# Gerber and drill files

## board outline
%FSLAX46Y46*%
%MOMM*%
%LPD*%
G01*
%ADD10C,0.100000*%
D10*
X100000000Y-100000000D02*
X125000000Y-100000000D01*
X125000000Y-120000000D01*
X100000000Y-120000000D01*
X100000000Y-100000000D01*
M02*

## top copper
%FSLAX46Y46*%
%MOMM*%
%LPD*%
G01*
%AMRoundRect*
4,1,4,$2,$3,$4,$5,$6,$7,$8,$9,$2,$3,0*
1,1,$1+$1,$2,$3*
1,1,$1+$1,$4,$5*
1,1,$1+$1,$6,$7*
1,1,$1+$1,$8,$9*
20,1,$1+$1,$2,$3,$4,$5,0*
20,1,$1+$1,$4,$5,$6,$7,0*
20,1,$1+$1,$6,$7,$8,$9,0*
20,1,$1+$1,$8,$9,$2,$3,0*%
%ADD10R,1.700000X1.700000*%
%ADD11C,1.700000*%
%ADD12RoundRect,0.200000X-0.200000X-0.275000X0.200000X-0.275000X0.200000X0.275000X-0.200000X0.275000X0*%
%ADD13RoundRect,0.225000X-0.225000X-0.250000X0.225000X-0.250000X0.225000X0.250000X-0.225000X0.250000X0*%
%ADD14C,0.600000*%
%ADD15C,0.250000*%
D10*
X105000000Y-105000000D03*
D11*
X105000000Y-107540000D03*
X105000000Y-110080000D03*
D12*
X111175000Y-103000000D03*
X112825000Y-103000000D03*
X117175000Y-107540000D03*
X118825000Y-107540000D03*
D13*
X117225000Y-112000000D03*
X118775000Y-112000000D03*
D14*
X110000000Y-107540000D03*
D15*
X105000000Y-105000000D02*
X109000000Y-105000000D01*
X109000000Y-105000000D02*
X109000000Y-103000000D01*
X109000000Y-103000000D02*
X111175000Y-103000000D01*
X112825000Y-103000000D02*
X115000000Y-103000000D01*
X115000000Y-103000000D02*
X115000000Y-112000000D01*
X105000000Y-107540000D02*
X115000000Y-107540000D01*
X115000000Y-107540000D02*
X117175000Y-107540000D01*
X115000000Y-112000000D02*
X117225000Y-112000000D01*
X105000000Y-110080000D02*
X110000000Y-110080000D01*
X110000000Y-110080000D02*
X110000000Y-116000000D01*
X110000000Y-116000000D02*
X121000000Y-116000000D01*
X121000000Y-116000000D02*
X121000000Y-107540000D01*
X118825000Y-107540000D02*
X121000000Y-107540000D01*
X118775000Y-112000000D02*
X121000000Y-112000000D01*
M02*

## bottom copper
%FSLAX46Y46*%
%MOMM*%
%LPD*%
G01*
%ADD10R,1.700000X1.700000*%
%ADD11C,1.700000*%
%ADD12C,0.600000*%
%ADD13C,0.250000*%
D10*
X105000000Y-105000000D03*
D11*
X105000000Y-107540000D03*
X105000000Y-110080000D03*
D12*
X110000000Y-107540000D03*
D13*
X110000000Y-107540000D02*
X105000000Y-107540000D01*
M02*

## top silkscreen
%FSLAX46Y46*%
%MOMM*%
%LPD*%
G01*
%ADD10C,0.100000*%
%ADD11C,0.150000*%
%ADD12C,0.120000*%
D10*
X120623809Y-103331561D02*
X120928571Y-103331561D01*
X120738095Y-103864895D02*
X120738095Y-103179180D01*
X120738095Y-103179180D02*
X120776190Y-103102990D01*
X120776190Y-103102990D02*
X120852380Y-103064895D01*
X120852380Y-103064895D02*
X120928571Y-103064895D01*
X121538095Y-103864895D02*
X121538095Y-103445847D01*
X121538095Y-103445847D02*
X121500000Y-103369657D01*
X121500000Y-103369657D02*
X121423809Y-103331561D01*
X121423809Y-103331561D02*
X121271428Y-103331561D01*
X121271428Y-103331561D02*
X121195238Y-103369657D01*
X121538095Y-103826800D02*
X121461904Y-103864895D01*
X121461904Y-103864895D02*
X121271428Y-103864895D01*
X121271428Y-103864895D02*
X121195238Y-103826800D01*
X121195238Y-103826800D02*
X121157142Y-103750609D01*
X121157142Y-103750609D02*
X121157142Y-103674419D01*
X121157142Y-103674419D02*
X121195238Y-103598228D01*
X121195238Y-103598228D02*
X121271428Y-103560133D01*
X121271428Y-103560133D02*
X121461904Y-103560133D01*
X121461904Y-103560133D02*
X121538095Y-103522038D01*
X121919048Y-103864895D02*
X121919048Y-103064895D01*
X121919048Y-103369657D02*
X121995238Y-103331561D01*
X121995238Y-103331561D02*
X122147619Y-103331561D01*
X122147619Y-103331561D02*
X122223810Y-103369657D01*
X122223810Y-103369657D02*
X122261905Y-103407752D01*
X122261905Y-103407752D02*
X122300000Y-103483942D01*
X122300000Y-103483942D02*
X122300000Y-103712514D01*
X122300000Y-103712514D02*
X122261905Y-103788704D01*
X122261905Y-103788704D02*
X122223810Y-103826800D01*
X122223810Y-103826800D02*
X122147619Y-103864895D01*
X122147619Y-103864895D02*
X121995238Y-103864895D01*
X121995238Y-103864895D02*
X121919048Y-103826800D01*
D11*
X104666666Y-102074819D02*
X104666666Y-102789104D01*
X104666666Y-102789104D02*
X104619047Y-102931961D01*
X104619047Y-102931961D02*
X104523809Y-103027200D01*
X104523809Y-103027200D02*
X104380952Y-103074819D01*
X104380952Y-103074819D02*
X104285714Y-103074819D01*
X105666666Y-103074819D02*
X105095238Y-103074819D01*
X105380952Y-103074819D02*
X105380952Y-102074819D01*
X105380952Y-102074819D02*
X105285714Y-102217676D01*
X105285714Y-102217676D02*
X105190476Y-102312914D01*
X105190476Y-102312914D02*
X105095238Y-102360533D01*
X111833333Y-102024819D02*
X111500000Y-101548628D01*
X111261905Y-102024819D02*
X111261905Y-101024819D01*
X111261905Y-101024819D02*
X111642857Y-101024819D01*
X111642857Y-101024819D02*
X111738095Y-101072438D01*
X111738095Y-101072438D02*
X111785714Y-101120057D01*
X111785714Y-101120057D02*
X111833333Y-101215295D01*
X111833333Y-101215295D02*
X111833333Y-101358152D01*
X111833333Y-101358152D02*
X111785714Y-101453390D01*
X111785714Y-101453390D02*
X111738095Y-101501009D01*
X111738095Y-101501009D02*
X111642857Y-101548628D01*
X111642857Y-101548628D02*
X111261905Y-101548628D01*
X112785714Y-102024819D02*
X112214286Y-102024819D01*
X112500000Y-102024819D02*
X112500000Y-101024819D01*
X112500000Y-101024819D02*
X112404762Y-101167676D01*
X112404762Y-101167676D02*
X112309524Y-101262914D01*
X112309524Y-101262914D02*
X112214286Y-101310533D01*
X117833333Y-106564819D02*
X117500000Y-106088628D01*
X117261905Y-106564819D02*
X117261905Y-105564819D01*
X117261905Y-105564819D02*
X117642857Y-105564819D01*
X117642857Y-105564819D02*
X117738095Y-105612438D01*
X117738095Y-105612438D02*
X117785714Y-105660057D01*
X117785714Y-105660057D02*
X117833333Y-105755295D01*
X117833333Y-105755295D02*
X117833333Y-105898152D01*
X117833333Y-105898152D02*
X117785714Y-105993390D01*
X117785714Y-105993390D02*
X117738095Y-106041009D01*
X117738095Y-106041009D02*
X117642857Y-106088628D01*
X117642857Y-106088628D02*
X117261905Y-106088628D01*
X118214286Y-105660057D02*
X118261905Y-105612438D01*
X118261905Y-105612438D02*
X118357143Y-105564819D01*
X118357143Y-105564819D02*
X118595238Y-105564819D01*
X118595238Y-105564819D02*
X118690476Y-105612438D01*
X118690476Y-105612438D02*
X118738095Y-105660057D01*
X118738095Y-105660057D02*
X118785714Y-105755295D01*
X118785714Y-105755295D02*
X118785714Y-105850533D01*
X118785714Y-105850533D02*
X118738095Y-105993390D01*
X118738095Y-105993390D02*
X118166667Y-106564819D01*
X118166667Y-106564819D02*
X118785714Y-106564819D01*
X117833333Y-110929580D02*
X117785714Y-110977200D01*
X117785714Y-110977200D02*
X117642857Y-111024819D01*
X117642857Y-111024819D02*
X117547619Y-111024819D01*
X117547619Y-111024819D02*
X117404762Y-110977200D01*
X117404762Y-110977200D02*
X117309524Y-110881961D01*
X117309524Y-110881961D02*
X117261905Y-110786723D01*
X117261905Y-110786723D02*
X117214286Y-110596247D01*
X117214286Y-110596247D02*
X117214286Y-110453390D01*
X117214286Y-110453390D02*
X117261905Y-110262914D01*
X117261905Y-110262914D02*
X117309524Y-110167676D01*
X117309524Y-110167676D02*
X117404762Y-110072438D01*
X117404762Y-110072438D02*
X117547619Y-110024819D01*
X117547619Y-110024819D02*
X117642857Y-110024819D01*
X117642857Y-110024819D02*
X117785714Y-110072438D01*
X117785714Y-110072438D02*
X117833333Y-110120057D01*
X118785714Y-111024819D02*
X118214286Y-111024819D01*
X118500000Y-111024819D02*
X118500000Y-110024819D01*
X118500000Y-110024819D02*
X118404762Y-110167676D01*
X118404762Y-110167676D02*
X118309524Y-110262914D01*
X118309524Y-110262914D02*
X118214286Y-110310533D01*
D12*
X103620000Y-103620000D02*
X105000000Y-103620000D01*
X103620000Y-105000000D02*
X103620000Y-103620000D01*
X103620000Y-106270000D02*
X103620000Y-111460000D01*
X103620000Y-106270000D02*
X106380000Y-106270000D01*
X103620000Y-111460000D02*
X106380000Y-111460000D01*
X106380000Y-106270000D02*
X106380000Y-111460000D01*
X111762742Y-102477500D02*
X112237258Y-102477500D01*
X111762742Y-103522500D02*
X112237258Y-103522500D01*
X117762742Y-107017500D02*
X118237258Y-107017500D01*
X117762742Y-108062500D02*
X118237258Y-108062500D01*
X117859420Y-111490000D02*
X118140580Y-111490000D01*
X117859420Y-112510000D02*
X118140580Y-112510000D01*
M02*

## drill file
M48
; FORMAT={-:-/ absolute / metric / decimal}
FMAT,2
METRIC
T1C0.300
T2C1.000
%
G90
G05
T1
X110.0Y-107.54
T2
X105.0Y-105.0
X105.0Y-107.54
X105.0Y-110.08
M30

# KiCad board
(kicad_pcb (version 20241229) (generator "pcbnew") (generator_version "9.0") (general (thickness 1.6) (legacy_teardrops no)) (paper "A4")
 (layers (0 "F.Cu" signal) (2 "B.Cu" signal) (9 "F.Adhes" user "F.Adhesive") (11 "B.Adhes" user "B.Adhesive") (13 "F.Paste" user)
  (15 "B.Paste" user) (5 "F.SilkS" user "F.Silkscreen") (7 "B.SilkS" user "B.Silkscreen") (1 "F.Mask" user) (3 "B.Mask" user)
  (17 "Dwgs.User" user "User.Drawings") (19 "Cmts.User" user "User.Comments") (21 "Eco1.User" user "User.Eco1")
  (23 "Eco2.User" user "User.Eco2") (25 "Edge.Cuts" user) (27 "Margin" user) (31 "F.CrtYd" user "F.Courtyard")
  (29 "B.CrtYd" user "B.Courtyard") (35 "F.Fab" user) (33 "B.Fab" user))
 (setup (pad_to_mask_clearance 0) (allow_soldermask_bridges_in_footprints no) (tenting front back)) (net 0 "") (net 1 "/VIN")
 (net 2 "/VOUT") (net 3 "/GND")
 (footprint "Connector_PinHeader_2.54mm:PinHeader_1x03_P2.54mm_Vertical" (layer "F.Cu") (at 105 105)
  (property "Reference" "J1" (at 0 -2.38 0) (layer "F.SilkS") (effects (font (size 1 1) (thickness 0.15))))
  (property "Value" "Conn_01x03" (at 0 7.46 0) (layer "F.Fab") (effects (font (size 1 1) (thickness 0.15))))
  (fp_line (start -1.38 -1.38) (end 0 -1.38) (stroke (width 0.12) (type solid)) (layer "F.SilkS"))
  (fp_line (start -1.38 0) (end -1.38 -1.38) (stroke (width 0.12) (type solid)) (layer "F.SilkS"))
  (fp_line (start -1.38 1.27) (end -1.38 6.46) (stroke (width 0.12) (type solid)) (layer "F.SilkS"))
  (fp_line (start -1.38 1.27) (end 1.38 1.27) (stroke (width 0.12) (type solid)) (layer "F.SilkS"))
  (fp_line (start -1.38 6.46) (end 1.38 6.46) (stroke (width 0.12) (type solid)) (layer "F.SilkS"))
  (fp_line (start 1.38 1.27) (end 1.38 6.46) (stroke (width 0.12) (type solid)) (layer "F.SilkS"))
  (pad "1" thru_hole rect (at 0 0) (size 1.7 1.7) (drill 1) (layers "*.Cu" "*.Mask") (remove_unused_layers no) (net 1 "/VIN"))
  (pad "2" thru_hole circle (at 0 2.54) (size 1.7 1.7) (drill 1) (layers "*.Cu" "*.Mask") (remove_unused_layers no) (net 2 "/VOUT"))
  (pad "3" thru_hole circle (at 0 5.08) (size 1.7 1.7) (drill 1) (layers "*.Cu" "*.Mask") (remove_unused_layers no) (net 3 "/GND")))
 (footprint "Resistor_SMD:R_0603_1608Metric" (layer "F.Cu") (at 112 103)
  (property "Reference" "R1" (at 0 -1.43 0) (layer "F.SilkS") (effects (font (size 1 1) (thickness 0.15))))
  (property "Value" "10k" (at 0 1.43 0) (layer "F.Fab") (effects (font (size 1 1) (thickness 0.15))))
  (fp_line (start -0.237258 -0.5225) (end 0.237258 -0.5225) (stroke (width 0.12) (type solid)) (layer "F.SilkS"))
  (fp_line (start -0.237258 0.5225) (end 0.237258 0.5225) (stroke (width 0.12) (type solid)) (layer "F.SilkS"))
  (pad "1" smd roundrect (at -0.825 0) (size 0.8 0.95) (layers "F.Cu" "F.Mask" "F.Paste") (roundrect_rratio 0.25) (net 1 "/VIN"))
  (pad "2" smd roundrect (at 0.825 0) (size 0.8 0.95) (layers "F.Cu" "F.Mask" "F.Paste") (roundrect_rratio 0.25) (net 2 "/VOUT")))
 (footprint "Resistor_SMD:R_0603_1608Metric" (layer "F.Cu") (at 118 107.54)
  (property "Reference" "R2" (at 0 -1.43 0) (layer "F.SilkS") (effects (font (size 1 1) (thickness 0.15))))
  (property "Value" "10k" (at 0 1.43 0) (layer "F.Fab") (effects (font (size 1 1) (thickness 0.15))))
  (fp_line (start -0.237258 -0.5225) (end 0.237258 -0.5225) (stroke (width 0.12) (type solid)) (layer "F.SilkS"))
  (fp_line (start -0.237258 0.5225) (end 0.237258 0.5225) (stroke (width 0.12) (type solid)) (layer "F.SilkS"))
  (pad "1" smd roundrect (at -0.825 0) (size 0.8 0.95) (layers "F.Cu" "F.Mask" "F.Paste") (roundrect_rratio 0.25) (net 2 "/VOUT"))
  (pad "2" smd roundrect (at 0.825 0) (size 0.8 0.95) (layers "F.Cu" "F.Mask" "F.Paste") (roundrect_rratio 0.25) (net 3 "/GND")))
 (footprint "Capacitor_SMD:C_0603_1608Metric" (layer "F.Cu") (at 118 112)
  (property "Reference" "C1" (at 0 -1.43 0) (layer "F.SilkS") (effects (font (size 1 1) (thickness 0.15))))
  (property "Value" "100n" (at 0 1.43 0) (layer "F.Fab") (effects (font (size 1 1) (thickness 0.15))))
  (fp_line (start -0.14058 -0.51) (end 0.14058 -0.51) (stroke (width 0.12) (type solid)) (layer "F.SilkS"))
  (fp_line (start -0.14058 0.51) (end 0.14058 0.51) (stroke (width 0.12) (type solid)) (layer "F.SilkS"))
  (pad "1" smd roundrect (at -0.775 0) (size 0.9 0.95) (layers "F.Cu" "F.Mask" "F.Paste") (roundrect_rratio 0.25) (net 2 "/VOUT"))
  (pad "2" smd roundrect (at 0.775 0) (size 0.9 0.95) (layers "F.Cu" "F.Mask" "F.Paste") (roundrect_rratio 0.25) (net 3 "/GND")))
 (gr_rect (start 100 100) (end 125 120) (stroke (width 0.1) (type default)) (fill no) (layer "Edge.Cuts"))
 (segment (start 105 105) (end 109 105) (width 0.25) (layer "F.Cu") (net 1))
 (segment (start 109 105) (end 109 103) (width 0.25) (layer "F.Cu") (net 1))
 (segment (start 109 103) (end 111.175 103) (width 0.25) (layer "F.Cu") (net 1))
 (segment (start 112.825 103) (end 115 103) (width 0.25) (layer "F.Cu") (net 2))
 (segment (start 115 103) (end 115 112) (width 0.25) (layer "F.Cu") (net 2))
 (segment (start 105 107.54) (end 115 107.54) (width 0.25) (layer "F.Cu") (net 2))
 (segment (start 115 107.54) (end 117.175 107.54) (width 0.25) (layer "F.Cu") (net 2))
 (segment (start 115 112) (end 117.225 112) (width 0.25) (layer "F.Cu") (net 2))
 (segment (start 105 110.08) (end 110 110.08) (width 0.25) (layer "F.Cu") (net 3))
 (segment (start 110 110.08) (end 110 116) (width 0.25) (layer "F.Cu") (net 3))
 (segment (start 110 116) (end 121 116) (width 0.25) (layer "F.Cu") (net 3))
 (segment (start 121 116) (end 121 107.54) (width 0.25) (layer "F.Cu") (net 3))
 (segment (start 118.825 107.54) (end 121 107.54) (width 0.25) (layer "F.Cu") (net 3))
 (segment (start 118.775 112) (end 121 112) (width 0.25) (layer "F.Cu") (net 3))
 (segment (start 110 107.54) (end 105 107.54) (width 0.25) (layer "B.Cu") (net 2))
 (via (at 110 107.54) (size 0.6) (drill 0.3) (layers "F.Cu" "B.Cu") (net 2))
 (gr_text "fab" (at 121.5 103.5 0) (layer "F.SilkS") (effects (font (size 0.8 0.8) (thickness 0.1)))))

